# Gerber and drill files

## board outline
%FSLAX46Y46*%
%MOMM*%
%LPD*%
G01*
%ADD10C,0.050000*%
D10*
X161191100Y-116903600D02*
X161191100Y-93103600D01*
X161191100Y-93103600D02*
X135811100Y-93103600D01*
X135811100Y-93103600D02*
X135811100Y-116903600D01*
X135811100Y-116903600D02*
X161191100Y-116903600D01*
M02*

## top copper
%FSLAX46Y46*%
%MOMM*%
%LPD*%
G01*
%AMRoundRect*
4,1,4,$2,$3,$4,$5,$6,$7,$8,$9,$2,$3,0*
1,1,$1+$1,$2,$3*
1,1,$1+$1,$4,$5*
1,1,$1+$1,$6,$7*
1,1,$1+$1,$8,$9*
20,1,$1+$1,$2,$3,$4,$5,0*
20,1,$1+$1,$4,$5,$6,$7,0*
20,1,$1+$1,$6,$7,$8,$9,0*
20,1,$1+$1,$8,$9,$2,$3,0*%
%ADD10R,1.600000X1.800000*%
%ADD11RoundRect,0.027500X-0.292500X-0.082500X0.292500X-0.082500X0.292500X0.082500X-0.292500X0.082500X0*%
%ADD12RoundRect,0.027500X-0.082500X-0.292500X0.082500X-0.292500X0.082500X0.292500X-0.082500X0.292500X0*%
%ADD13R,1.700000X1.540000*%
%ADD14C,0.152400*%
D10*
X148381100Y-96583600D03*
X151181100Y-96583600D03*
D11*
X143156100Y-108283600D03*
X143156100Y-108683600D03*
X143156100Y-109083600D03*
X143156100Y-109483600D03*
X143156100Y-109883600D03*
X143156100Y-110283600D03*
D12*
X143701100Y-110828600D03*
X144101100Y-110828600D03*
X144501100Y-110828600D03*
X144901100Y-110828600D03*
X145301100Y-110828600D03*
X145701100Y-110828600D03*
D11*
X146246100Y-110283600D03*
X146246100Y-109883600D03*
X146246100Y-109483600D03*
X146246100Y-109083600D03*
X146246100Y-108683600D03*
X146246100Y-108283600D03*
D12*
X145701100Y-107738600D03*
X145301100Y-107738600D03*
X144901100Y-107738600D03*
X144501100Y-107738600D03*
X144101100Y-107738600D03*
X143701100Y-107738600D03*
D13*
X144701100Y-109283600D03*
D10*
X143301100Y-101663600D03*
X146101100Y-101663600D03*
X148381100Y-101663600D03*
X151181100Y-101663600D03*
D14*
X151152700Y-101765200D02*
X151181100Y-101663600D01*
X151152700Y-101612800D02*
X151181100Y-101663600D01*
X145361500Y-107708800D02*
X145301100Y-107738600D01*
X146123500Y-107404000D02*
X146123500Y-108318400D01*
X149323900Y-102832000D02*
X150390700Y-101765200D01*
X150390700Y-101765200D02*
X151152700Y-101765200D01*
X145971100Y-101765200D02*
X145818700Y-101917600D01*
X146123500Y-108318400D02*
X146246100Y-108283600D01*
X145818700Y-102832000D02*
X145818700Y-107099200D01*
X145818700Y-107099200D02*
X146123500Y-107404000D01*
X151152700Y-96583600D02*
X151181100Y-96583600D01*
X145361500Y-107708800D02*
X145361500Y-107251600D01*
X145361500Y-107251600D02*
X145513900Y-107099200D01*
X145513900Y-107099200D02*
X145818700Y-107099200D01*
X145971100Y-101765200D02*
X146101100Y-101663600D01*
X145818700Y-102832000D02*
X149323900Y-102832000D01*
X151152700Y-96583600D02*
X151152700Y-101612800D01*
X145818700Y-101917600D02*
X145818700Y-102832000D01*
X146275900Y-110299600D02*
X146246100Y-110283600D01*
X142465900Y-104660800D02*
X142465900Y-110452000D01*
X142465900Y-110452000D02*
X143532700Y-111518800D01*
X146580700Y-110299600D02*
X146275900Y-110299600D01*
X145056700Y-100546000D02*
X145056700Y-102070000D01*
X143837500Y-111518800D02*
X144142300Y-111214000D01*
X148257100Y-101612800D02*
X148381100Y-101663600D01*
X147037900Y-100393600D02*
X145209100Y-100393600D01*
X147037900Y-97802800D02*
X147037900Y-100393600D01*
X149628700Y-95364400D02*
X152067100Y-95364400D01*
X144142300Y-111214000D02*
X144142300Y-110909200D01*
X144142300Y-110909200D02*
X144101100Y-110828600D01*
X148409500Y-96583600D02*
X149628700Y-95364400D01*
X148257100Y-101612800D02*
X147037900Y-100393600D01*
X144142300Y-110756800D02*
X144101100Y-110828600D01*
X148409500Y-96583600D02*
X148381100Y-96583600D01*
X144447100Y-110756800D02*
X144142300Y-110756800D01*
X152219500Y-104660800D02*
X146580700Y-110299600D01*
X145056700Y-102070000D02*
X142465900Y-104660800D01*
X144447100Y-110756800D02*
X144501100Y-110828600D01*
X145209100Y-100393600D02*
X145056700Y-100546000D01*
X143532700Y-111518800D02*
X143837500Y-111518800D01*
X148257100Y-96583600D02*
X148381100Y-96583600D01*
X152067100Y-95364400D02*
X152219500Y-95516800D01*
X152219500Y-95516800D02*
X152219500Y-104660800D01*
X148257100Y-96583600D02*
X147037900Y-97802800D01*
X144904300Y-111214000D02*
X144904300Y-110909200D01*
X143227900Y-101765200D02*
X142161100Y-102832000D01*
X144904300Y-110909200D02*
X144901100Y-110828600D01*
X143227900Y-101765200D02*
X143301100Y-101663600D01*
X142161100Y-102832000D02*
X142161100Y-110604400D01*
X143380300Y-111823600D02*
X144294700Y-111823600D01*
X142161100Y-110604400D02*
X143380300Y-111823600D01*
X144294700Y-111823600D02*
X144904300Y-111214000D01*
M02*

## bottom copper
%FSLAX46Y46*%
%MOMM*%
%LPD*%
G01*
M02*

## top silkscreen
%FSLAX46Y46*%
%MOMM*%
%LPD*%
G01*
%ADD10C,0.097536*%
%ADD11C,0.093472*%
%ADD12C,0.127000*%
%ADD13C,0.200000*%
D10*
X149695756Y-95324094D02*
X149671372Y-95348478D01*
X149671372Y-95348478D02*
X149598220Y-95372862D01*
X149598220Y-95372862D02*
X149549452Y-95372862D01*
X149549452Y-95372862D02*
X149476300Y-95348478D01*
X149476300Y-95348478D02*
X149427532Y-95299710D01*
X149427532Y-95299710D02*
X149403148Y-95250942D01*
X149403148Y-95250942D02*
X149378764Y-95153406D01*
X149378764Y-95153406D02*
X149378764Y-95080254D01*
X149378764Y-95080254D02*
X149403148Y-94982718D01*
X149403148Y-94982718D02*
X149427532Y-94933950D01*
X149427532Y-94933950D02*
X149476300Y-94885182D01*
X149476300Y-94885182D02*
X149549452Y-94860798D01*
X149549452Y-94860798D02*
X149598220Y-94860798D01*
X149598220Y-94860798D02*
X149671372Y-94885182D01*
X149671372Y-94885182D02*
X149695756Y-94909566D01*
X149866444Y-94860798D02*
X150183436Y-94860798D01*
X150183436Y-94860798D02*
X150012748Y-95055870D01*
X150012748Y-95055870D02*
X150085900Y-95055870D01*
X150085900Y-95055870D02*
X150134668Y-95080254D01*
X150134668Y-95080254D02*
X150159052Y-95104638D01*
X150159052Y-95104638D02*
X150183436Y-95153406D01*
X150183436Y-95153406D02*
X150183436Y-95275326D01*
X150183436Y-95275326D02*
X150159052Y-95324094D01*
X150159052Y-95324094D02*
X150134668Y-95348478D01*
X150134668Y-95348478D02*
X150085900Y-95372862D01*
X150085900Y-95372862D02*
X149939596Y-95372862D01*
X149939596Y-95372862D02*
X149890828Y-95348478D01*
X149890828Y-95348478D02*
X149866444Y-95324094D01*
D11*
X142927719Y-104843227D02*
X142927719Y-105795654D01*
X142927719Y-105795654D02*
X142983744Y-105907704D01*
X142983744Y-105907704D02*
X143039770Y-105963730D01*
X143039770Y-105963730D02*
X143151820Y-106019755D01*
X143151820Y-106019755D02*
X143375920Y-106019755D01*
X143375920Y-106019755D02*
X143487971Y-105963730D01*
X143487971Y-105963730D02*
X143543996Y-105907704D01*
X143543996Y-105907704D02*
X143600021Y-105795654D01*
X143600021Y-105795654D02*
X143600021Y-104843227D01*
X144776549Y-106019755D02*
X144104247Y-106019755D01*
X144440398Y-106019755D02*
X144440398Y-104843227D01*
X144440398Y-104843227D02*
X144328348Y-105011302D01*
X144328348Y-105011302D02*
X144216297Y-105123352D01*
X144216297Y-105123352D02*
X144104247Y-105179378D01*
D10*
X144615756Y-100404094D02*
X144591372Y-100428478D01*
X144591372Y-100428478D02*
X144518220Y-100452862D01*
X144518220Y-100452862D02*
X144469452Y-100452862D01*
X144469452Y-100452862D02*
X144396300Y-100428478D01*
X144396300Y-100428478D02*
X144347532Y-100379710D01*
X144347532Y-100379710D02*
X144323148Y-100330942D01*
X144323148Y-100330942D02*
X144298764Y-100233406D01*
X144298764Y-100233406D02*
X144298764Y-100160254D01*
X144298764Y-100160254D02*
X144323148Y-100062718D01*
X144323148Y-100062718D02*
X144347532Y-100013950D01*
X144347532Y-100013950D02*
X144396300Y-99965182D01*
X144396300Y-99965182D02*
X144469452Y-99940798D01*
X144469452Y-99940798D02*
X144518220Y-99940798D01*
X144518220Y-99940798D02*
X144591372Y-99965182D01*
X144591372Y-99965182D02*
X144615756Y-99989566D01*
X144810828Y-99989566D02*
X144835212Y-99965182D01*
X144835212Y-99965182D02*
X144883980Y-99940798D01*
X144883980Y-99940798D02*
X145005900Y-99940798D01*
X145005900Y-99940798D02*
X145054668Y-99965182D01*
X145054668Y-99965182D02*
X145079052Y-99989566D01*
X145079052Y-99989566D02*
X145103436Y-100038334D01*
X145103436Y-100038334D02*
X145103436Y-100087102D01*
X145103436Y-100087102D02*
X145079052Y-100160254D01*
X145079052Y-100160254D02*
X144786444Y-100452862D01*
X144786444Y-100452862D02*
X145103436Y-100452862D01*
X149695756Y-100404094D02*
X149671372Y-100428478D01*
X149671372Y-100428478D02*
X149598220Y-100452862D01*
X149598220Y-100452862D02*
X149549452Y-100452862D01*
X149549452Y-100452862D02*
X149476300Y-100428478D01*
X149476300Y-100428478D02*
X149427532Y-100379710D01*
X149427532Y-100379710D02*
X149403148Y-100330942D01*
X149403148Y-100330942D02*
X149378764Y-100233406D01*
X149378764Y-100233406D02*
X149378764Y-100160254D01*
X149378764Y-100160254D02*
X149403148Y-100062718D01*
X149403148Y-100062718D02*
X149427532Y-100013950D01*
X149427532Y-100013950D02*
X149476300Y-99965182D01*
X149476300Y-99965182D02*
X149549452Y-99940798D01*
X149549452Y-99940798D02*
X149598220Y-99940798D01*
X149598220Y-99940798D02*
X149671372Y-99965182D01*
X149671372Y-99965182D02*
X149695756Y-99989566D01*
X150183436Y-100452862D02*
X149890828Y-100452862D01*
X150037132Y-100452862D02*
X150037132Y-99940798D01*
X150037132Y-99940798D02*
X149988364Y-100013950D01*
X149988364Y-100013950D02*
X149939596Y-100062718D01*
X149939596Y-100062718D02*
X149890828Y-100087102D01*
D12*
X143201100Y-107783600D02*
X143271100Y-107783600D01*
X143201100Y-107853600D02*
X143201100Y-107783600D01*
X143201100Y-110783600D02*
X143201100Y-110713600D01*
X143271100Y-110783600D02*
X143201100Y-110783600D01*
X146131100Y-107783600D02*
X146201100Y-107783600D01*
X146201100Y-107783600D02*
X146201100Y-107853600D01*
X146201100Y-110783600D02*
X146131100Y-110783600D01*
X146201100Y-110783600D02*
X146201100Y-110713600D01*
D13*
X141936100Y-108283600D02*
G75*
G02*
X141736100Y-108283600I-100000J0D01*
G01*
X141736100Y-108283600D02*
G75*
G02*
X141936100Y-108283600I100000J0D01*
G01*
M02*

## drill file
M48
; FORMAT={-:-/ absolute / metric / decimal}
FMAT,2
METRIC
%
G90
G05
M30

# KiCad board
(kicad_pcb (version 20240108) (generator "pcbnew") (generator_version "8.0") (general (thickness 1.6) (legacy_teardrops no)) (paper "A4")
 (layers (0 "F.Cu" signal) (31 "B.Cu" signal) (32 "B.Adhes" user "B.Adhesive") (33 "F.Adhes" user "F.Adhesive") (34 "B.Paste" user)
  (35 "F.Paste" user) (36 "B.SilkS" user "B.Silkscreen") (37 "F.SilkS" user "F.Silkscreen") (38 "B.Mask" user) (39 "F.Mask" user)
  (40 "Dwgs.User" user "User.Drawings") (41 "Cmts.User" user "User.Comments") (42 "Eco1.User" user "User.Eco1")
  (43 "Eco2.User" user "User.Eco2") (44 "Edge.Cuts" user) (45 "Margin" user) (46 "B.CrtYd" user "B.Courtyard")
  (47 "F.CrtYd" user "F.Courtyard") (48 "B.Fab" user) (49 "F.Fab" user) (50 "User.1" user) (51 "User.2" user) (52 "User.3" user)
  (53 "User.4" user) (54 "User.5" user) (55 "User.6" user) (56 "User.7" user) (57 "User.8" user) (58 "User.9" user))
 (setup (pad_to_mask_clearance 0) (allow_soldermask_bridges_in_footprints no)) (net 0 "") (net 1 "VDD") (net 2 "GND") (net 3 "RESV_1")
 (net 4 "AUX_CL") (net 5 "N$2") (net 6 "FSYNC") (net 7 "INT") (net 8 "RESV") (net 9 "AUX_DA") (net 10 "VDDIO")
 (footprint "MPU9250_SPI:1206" (layer "F.Cu") (at 149.7811 96.5836)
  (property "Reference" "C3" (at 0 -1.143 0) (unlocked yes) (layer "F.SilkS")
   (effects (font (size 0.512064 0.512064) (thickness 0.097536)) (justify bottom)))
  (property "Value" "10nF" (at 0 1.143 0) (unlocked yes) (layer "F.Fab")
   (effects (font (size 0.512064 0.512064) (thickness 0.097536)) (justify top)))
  (pad "1" smd rect (at -1.4 0) (size 1.6 1.8) (layers "F.Cu" "F.Paste" "F.Mask") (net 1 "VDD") (solder_mask_margin 0.1016)
   (thermal_bridge_angle 0))
  (pad "2" smd rect (at 1.4 0) (size 1.6 1.8) (layers "F.Cu" "F.Paste" "F.Mask") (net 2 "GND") (solder_mask_margin 0.1016)
   (thermal_bridge_angle 0)))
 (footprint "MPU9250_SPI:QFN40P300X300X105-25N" (layer "F.Cu") (at 144.7011 109.2836)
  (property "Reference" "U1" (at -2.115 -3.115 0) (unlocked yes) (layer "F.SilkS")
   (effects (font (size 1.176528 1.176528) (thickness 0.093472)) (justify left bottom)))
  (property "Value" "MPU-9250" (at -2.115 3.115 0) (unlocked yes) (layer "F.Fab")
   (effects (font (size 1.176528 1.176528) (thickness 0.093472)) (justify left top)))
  (fp_line (start -1.5 -1.5) (end -1.43 -1.5) (stroke (width 0.127) (type solid)) (layer "F.SilkS"))
  (fp_line (start -1.5 -1.43) (end -1.5 -1.5) (stroke (width 0.127) (type solid)) (layer "F.SilkS"))
  (fp_line (start -1.5 1.5) (end -1.5 1.43) (stroke (width 0.127) (type solid)) (layer "F.SilkS"))
  (fp_line (start -1.43 1.5) (end -1.5 1.5) (stroke (width 0.127) (type solid)) (layer "F.SilkS"))
  (fp_line (start 1.43 -1.5) (end 1.5 -1.5) (stroke (width 0.127) (type solid)) (layer "F.SilkS"))
  (fp_line (start 1.5 -1.5) (end 1.5 -1.43) (stroke (width 0.127) (type solid)) (layer "F.SilkS"))
  (fp_line (start 1.5 1.5) (end 1.43 1.5) (stroke (width 0.127) (type solid)) (layer "F.SilkS"))
  (fp_line (start 1.5 1.5) (end 1.5 1.43) (stroke (width 0.127) (type solid)) (layer "F.SilkS"))
  (fp_circle (center -2.865 -1) (end -2.765 -1) (stroke (width 0.2) (type solid)) (fill none) (layer "F.SilkS"))
  (pad "1" smd roundrect (at -1.545 -1) (size 0.64 0.22) (layers "F.Cu" "F.Paste" "F.Mask") (roundrect_rratio 0.125) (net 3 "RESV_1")
   (solder_mask_margin 0.1016) (thermal_bridge_angle 0))
  (pad "2" smd roundrect (at -1.545 -0.6) (size 0.64 0.22) (layers "F.Cu" "F.Paste" "F.Mask") (roundrect_rratio 0.125)
   (solder_mask_margin 0.1016) (thermal_bridge_angle 0))
  (pad "3" smd roundrect (at -1.545 -0.2) (size 0.64 0.22) (layers "F.Cu" "F.Paste" "F.Mask") (roundrect_rratio 0.125)
   (solder_mask_margin 0.1016) (thermal_bridge_angle 0))
  (pad "4" smd roundrect (at -1.545 0.2) (size 0.64 0.22) (layers "F.Cu" "F.Paste" "F.Mask") (roundrect_rratio 0.125)
   (solder_mask_margin 0.1016) (thermal_bridge_angle 0))
  (pad "5" smd roundrect (at -1.545 0.6) (size 0.64 0.22) (layers "F.Cu" "F.Paste" "F.Mask") (roundrect_rratio 0.125)
   (solder_mask_margin 0.1016) (thermal_bridge_angle 0))
  (pad "6" smd roundrect (at -1.545 1) (size 0.64 0.22) (layers "F.Cu" "F.Paste" "F.Mask") (roundrect_rratio 0.125)
   (solder_mask_margin 0.1016) (thermal_bridge_angle 0))
  (pad "7" smd roundrect (at -1 1.545) (size 0.22 0.64) (layers "F.Cu" "F.Paste" "F.Mask") (roundrect_rratio 0.125) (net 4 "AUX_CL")
   (solder_mask_margin 0.1016) (thermal_bridge_angle 0))
  (pad "8" smd roundrect (at -0.6 1.545) (size 0.22 0.64) (layers "F.Cu" "F.Paste" "F.Mask") (roundrect_rratio 0.125) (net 1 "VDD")
   (solder_mask_margin 0.1016) (thermal_bridge_angle 0))
  (pad "9" smd roundrect (at -0.2 1.545) (size 0.22 0.64) (layers "F.Cu" "F.Paste" "F.Mask") (roundrect_rratio 0.125) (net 1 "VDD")
   (solder_mask_margin 0.1016) (thermal_bridge_angle 0))
  (pad "10" smd roundrect (at 0.2 1.545) (size 0.22 0.64) (layers "F.Cu" "F.Paste" "F.Mask") (roundrect_rratio 0.125) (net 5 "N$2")
   (solder_mask_margin 0.1016) (thermal_bridge_angle 0))
  (pad "11" smd roundrect (at 0.6 1.545) (size 0.22 0.64) (layers "F.Cu" "F.Paste" "F.Mask") (roundrect_rratio 0.125) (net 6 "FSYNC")
   (solder_mask_margin 0.1016) (thermal_bridge_angle 0))
  (pad "12" smd roundrect (at 1 1.545) (size 0.22 0.64) (layers "F.Cu" "F.Paste" "F.Mask") (roundrect_rratio 0.125) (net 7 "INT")
   (solder_mask_margin 0.1016) (thermal_bridge_angle 0))
  (pad "13" smd roundrect (at 1.545 1) (size 0.64 0.22) (layers "F.Cu" "F.Paste" "F.Mask") (roundrect_rratio 0.125) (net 1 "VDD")
   (solder_mask_margin 0.1016) (thermal_bridge_angle 0))
  (pad "14" smd roundrect (at 1.545 0.6) (size 0.64 0.22) (layers "F.Cu" "F.Paste" "F.Mask") (roundrect_rratio 0.125)
   (solder_mask_margin 0.1016) (thermal_bridge_angle 0))
  (pad "15" smd roundrect (at 1.545 0.2) (size 0.64 0.22) (layers "F.Cu" "F.Paste" "F.Mask") (roundrect_rratio 0.125)
   (solder_mask_margin 0.1016) (thermal_bridge_angle 0))
  (pad "16" smd roundrect (at 1.545 -0.2) (size 0.64 0.22) (layers "F.Cu" "F.Paste" "F.Mask") (roundrect_rratio 0.125)
   (solder_mask_margin 0.1016) (thermal_bridge_angle 0))
  (pad "17" smd roundrect (at 1.545 -0.6) (size 0.64 0.22) (layers "F.Cu" "F.Paste" "F.Mask") (roundrect_rratio 0.125)
   (solder_mask_margin 0.1016) (thermal_bridge_angle 0))
  (pad "18" smd roundrect (at 1.545 -1) (size 0.64 0.22) (layers "F.Cu" "F.Paste" "F.Mask") (roundrect_rratio 0.125) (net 2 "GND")
   (solder_mask_margin 0.1016) (thermal_bridge_angle 0))
  (pad "19" smd roundrect (at 1 -1.545) (size 0.22 0.64) (layers "F.Cu" "F.Paste" "F.Mask") (roundrect_rratio 0.125) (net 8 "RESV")
   (solder_mask_margin 0.1016) (thermal_bridge_angle 0))
  (pad "20" smd roundrect (at 0.6 -1.545) (size 0.22 0.64) (layers "F.Cu" "F.Paste" "F.Mask") (roundrect_rratio 0.125) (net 2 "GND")
   (solder_mask_margin 0.1016) (thermal_bridge_angle 0))
  (pad "21" smd roundrect (at 0.2 -1.545) (size 0.22 0.64) (layers "F.Cu" "F.Paste" "F.Mask") (roundrect_rratio 0.125) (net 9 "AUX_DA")
   (solder_mask_margin 0.1016) (thermal_bridge_angle 0))
  (pad "22" smd roundrect (at -0.2 -1.545) (size 0.22 0.64) (layers "F.Cu" "F.Paste" "F.Mask") (roundrect_rratio 0.125) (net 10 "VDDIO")
   (solder_mask_margin 0.1016) (thermal_bridge_angle 0))
  (pad "23" smd roundrect (at -0.6 -1.545) (size 0.22 0.64) (layers "F.Cu" "F.Paste" "F.Mask") (roundrect_rratio 0.125)
   (solder_mask_margin 0.1016) (thermal_bridge_angle 0))
  (pad "24" smd roundrect (at -1 -1.545) (size 0.22 0.64) (layers "F.Cu" "F.Paste" "F.Mask") (roundrect_rratio 0.125)
   (solder_mask_margin 0.1016) (thermal_bridge_angle 0))
  (pad "25" smd rect (at 0 0) (size 1.7 1.54) (layers "F.Cu" "F.Mask") (solder_mask_margin 0.1016) (thermal_bridge_angle 0)))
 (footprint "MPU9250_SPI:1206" (layer "F.Cu") (at 144.7011 101.6636)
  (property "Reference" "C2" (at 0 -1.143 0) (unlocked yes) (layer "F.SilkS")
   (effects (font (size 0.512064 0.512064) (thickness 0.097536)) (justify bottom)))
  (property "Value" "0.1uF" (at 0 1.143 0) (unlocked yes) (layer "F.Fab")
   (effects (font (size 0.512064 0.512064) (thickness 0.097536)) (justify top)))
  (pad "1" smd rect (at -1.4 0) (size 1.6 1.8) (layers "F.Cu" "F.Paste" "F.Mask") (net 5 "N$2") (solder_mask_margin 0.1016)
   (thermal_bridge_angle 0))
  (pad "2" smd rect (at 1.4 0) (size 1.6 1.8) (layers "F.Cu" "F.Paste" "F.Mask") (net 2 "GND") (solder_mask_margin 0.1016)
   (thermal_bridge_angle 0)))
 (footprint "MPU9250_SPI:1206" (layer "F.Cu") (at 149.7811 101.6636)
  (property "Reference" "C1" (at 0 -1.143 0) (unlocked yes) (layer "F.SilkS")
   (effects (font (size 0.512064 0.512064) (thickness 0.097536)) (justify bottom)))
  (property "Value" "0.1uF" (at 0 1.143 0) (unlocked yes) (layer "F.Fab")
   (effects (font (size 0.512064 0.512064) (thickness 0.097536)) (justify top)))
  (pad "1" smd rect (at -1.4 0) (size 1.6 1.8) (layers "F.Cu" "F.Paste" "F.Mask") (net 1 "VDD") (solder_mask_margin 0.1016)
   (thermal_bridge_angle 0))
  (pad "2" smd rect (at 1.4 0) (size 1.6 1.8) (layers "F.Cu" "F.Paste" "F.Mask") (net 2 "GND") (solder_mask_margin 0.1016)
   (thermal_bridge_angle 0)))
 (gr_line (start 161.1911 116.9036) (end 161.1911 93.1036) (stroke (width 0.05) (type solid)) (layer "Edge.Cuts"))
 (gr_line (start 161.1911 93.1036) (end 135.8111 93.1036) (stroke (width 0.05) (type solid)) (layer "Edge.Cuts"))
 (gr_line (start 135.8111 93.1036) (end 135.8111 116.9036) (stroke (width 0.05) (type solid)) (layer "Edge.Cuts"))
 (gr_line (start 135.8111 116.9036) (end 161.1911 116.9036) (stroke (width 0.05) (type solid)) (layer "Edge.Cuts"))
 (segment (start 151.1527 101.7652) (end 151.1811 101.6636) (width 0.1524) (layer "F.Cu") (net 2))
 (segment (start 151.1527 101.6128) (end 151.1811 101.6636) (width 0.1524) (layer "F.Cu") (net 2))
 (segment (start 145.3615 107.7088) (end 145.3011 107.7386) (width 0.1524) (layer "F.Cu") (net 2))
 (segment (start 146.1235 107.404) (end 146.1235 108.3184) (width 0.1524) (layer "F.Cu") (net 2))
 (segment (start 149.3239 102.832) (end 150.3907 101.7652) (width 0.1524) (layer "F.Cu") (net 2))
 (segment (start 150.3907 101.7652) (end 151.1527 101.7652) (width 0.1524) (layer "F.Cu") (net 2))
 (segment (start 145.9711 101.7652) (end 145.8187 101.9176) (width 0.1524) (layer "F.Cu") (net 2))
 (segment (start 146.1235 108.3184) (end 146.2461 108.2836) (width 0.1524) (layer "F.Cu") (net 2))
 (segment (start 145.8187 102.832) (end 145.8187 107.0992) (width 0.1524) (layer "F.Cu") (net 2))
 (segment (start 145.8187 107.0992) (end 146.1235 107.404) (width 0.1524) (layer "F.Cu") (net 2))
 (segment (start 151.1527 96.5836) (end 151.1811 96.5836) (width 0.1524) (layer "F.Cu") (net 2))
 (segment (start 145.3615 107.7088) (end 145.3615 107.2516) (width 0.1524) (layer "F.Cu") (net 2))
 (segment (start 145.3615 107.2516) (end 145.5139 107.0992) (width 0.1524) (layer "F.Cu") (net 2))
 (segment (start 145.5139 107.0992) (end 145.8187 107.0992) (width 0.1524) (layer "F.Cu") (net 2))
 (segment (start 145.9711 101.7652) (end 146.1011 101.6636) (width 0.1524) (layer "F.Cu") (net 2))
 (segment (start 145.8187 102.832) (end 149.3239 102.832) (width 0.1524) (layer "F.Cu") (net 2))
 (segment (start 151.1527 96.5836) (end 151.1527 101.6128) (width 0.1524) (layer "F.Cu") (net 2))
 (segment (start 145.8187 101.9176) (end 145.8187 102.832) (width 0.1524) (layer "F.Cu") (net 2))
 (segment (start 146.2759 110.2996) (end 146.2461 110.2836) (width 0.1524) (layer "F.Cu") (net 1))
 (segment (start 142.4659 104.6608) (end 142.4659 110.452) (width 0.1524) (layer "F.Cu") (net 1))
 (segment (start 142.4659 110.452) (end 143.5327 111.5188) (width 0.1524) (layer "F.Cu") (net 1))
 (segment (start 146.5807 110.2996) (end 146.2759 110.2996) (width 0.1524) (layer "F.Cu") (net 1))
 (segment (start 145.0567 100.546) (end 145.0567 102.07) (width 0.1524) (layer "F.Cu") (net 1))
 (segment (start 143.8375 111.5188) (end 144.1423 111.214) (width 0.1524) (layer "F.Cu") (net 1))
 (segment (start 148.2571 101.6128) (end 148.3811 101.6636) (width 0.1524) (layer "F.Cu") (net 1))
 (segment (start 147.0379 100.3936) (end 145.2091 100.3936) (width 0.1524) (layer "F.Cu") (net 1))
 (segment (start 147.0379 97.8028) (end 147.0379 100.3936) (width 0.1524) (layer "F.Cu") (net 1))
 (segment (start 149.6287 95.3644) (end 152.0671 95.3644) (width 0.1524) (layer "F.Cu") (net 1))
 (segment (start 144.1423 111.214) (end 144.1423 110.9092) (width 0.1524) (layer "F.Cu") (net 1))
 (segment (start 144.1423 110.9092) (end 144.1011 110.8286) (width 0.1524) (layer "F.Cu") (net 1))
 (segment (start 148.4095 96.5836) (end 149.6287 95.3644) (width 0.1524) (layer "F.Cu") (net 1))
 (segment (start 148.2571 101.6128) (end 147.0379 100.3936) (width 0.1524) (layer "F.Cu") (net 1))
 (segment (start 144.1423 110.7568) (end 144.1011 110.8286) (width 0.1524) (layer "F.Cu") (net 1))
 (segment (start 148.4095 96.5836) (end 148.3811 96.5836) (width 0.1524) (layer "F.Cu") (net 1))
 (segment (start 144.4471 110.7568) (end 144.1423 110.7568) (width 0.1524) (layer "F.Cu") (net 1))
 (segment (start 152.2195 104.6608) (end 146.5807 110.2996) (width 0.1524) (layer "F.Cu") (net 1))
 (segment (start 145.0567 102.07) (end 142.4659 104.6608) (width 0.1524) (layer "F.Cu") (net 1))
 (segment (start 144.4471 110.7568) (end 144.5011 110.8286) (width 0.1524) (layer "F.Cu") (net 1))
 (segment (start 145.2091 100.3936) (end 145.0567 100.546) (width 0.1524) (layer "F.Cu") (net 1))
 (segment (start 143.5327 111.5188) (end 143.8375 111.5188) (width 0.1524) (layer "F.Cu") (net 1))
 (segment (start 148.2571 96.5836) (end 148.3811 96.5836) (width 0.1524) (layer "F.Cu") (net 1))
 (segment (start 152.0671 95.3644) (end 152.2195 95.5168) (width 0.1524) (layer "F.Cu") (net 1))
 (segment (start 152.2195 95.5168) (end 152.2195 104.6608) (width 0.1524) (layer "F.Cu") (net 1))
 (segment (start 148.2571 96.5836) (end 147.0379 97.8028) (width 0.1524) (layer "F.Cu") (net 1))
 (segment (start 144.9043 111.214) (end 144.9043 110.9092) (width 0.1524) (layer "F.Cu") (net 5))
 (segment (start 143.2279 101.7652) (end 142.1611 102.832) (width 0.1524) (layer "F.Cu") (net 5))
 (segment (start 144.9043 110.9092) (end 144.9011 110.8286) (width 0.1524) (layer "F.Cu") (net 5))
 (segment (start 143.2279 101.7652) (end 143.3011 101.6636) (width 0.1524) (layer "F.Cu") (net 5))
 (segment (start 142.1611 102.832) (end 142.1611 110.6044) (width 0.1524) (layer "F.Cu") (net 5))
 (segment (start 143.3803 111.8236) (end 144.2947 111.8236) (width 0.1524) (layer "F.Cu") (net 5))
 (segment (start 142.1611 110.6044) (end 143.3803 111.8236) (width 0.1524) (layer "F.Cu") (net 5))
 (segment (start 144.2947 111.8236) (end 144.9043 111.214) (width 0.1524) (layer "F.Cu") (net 5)))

